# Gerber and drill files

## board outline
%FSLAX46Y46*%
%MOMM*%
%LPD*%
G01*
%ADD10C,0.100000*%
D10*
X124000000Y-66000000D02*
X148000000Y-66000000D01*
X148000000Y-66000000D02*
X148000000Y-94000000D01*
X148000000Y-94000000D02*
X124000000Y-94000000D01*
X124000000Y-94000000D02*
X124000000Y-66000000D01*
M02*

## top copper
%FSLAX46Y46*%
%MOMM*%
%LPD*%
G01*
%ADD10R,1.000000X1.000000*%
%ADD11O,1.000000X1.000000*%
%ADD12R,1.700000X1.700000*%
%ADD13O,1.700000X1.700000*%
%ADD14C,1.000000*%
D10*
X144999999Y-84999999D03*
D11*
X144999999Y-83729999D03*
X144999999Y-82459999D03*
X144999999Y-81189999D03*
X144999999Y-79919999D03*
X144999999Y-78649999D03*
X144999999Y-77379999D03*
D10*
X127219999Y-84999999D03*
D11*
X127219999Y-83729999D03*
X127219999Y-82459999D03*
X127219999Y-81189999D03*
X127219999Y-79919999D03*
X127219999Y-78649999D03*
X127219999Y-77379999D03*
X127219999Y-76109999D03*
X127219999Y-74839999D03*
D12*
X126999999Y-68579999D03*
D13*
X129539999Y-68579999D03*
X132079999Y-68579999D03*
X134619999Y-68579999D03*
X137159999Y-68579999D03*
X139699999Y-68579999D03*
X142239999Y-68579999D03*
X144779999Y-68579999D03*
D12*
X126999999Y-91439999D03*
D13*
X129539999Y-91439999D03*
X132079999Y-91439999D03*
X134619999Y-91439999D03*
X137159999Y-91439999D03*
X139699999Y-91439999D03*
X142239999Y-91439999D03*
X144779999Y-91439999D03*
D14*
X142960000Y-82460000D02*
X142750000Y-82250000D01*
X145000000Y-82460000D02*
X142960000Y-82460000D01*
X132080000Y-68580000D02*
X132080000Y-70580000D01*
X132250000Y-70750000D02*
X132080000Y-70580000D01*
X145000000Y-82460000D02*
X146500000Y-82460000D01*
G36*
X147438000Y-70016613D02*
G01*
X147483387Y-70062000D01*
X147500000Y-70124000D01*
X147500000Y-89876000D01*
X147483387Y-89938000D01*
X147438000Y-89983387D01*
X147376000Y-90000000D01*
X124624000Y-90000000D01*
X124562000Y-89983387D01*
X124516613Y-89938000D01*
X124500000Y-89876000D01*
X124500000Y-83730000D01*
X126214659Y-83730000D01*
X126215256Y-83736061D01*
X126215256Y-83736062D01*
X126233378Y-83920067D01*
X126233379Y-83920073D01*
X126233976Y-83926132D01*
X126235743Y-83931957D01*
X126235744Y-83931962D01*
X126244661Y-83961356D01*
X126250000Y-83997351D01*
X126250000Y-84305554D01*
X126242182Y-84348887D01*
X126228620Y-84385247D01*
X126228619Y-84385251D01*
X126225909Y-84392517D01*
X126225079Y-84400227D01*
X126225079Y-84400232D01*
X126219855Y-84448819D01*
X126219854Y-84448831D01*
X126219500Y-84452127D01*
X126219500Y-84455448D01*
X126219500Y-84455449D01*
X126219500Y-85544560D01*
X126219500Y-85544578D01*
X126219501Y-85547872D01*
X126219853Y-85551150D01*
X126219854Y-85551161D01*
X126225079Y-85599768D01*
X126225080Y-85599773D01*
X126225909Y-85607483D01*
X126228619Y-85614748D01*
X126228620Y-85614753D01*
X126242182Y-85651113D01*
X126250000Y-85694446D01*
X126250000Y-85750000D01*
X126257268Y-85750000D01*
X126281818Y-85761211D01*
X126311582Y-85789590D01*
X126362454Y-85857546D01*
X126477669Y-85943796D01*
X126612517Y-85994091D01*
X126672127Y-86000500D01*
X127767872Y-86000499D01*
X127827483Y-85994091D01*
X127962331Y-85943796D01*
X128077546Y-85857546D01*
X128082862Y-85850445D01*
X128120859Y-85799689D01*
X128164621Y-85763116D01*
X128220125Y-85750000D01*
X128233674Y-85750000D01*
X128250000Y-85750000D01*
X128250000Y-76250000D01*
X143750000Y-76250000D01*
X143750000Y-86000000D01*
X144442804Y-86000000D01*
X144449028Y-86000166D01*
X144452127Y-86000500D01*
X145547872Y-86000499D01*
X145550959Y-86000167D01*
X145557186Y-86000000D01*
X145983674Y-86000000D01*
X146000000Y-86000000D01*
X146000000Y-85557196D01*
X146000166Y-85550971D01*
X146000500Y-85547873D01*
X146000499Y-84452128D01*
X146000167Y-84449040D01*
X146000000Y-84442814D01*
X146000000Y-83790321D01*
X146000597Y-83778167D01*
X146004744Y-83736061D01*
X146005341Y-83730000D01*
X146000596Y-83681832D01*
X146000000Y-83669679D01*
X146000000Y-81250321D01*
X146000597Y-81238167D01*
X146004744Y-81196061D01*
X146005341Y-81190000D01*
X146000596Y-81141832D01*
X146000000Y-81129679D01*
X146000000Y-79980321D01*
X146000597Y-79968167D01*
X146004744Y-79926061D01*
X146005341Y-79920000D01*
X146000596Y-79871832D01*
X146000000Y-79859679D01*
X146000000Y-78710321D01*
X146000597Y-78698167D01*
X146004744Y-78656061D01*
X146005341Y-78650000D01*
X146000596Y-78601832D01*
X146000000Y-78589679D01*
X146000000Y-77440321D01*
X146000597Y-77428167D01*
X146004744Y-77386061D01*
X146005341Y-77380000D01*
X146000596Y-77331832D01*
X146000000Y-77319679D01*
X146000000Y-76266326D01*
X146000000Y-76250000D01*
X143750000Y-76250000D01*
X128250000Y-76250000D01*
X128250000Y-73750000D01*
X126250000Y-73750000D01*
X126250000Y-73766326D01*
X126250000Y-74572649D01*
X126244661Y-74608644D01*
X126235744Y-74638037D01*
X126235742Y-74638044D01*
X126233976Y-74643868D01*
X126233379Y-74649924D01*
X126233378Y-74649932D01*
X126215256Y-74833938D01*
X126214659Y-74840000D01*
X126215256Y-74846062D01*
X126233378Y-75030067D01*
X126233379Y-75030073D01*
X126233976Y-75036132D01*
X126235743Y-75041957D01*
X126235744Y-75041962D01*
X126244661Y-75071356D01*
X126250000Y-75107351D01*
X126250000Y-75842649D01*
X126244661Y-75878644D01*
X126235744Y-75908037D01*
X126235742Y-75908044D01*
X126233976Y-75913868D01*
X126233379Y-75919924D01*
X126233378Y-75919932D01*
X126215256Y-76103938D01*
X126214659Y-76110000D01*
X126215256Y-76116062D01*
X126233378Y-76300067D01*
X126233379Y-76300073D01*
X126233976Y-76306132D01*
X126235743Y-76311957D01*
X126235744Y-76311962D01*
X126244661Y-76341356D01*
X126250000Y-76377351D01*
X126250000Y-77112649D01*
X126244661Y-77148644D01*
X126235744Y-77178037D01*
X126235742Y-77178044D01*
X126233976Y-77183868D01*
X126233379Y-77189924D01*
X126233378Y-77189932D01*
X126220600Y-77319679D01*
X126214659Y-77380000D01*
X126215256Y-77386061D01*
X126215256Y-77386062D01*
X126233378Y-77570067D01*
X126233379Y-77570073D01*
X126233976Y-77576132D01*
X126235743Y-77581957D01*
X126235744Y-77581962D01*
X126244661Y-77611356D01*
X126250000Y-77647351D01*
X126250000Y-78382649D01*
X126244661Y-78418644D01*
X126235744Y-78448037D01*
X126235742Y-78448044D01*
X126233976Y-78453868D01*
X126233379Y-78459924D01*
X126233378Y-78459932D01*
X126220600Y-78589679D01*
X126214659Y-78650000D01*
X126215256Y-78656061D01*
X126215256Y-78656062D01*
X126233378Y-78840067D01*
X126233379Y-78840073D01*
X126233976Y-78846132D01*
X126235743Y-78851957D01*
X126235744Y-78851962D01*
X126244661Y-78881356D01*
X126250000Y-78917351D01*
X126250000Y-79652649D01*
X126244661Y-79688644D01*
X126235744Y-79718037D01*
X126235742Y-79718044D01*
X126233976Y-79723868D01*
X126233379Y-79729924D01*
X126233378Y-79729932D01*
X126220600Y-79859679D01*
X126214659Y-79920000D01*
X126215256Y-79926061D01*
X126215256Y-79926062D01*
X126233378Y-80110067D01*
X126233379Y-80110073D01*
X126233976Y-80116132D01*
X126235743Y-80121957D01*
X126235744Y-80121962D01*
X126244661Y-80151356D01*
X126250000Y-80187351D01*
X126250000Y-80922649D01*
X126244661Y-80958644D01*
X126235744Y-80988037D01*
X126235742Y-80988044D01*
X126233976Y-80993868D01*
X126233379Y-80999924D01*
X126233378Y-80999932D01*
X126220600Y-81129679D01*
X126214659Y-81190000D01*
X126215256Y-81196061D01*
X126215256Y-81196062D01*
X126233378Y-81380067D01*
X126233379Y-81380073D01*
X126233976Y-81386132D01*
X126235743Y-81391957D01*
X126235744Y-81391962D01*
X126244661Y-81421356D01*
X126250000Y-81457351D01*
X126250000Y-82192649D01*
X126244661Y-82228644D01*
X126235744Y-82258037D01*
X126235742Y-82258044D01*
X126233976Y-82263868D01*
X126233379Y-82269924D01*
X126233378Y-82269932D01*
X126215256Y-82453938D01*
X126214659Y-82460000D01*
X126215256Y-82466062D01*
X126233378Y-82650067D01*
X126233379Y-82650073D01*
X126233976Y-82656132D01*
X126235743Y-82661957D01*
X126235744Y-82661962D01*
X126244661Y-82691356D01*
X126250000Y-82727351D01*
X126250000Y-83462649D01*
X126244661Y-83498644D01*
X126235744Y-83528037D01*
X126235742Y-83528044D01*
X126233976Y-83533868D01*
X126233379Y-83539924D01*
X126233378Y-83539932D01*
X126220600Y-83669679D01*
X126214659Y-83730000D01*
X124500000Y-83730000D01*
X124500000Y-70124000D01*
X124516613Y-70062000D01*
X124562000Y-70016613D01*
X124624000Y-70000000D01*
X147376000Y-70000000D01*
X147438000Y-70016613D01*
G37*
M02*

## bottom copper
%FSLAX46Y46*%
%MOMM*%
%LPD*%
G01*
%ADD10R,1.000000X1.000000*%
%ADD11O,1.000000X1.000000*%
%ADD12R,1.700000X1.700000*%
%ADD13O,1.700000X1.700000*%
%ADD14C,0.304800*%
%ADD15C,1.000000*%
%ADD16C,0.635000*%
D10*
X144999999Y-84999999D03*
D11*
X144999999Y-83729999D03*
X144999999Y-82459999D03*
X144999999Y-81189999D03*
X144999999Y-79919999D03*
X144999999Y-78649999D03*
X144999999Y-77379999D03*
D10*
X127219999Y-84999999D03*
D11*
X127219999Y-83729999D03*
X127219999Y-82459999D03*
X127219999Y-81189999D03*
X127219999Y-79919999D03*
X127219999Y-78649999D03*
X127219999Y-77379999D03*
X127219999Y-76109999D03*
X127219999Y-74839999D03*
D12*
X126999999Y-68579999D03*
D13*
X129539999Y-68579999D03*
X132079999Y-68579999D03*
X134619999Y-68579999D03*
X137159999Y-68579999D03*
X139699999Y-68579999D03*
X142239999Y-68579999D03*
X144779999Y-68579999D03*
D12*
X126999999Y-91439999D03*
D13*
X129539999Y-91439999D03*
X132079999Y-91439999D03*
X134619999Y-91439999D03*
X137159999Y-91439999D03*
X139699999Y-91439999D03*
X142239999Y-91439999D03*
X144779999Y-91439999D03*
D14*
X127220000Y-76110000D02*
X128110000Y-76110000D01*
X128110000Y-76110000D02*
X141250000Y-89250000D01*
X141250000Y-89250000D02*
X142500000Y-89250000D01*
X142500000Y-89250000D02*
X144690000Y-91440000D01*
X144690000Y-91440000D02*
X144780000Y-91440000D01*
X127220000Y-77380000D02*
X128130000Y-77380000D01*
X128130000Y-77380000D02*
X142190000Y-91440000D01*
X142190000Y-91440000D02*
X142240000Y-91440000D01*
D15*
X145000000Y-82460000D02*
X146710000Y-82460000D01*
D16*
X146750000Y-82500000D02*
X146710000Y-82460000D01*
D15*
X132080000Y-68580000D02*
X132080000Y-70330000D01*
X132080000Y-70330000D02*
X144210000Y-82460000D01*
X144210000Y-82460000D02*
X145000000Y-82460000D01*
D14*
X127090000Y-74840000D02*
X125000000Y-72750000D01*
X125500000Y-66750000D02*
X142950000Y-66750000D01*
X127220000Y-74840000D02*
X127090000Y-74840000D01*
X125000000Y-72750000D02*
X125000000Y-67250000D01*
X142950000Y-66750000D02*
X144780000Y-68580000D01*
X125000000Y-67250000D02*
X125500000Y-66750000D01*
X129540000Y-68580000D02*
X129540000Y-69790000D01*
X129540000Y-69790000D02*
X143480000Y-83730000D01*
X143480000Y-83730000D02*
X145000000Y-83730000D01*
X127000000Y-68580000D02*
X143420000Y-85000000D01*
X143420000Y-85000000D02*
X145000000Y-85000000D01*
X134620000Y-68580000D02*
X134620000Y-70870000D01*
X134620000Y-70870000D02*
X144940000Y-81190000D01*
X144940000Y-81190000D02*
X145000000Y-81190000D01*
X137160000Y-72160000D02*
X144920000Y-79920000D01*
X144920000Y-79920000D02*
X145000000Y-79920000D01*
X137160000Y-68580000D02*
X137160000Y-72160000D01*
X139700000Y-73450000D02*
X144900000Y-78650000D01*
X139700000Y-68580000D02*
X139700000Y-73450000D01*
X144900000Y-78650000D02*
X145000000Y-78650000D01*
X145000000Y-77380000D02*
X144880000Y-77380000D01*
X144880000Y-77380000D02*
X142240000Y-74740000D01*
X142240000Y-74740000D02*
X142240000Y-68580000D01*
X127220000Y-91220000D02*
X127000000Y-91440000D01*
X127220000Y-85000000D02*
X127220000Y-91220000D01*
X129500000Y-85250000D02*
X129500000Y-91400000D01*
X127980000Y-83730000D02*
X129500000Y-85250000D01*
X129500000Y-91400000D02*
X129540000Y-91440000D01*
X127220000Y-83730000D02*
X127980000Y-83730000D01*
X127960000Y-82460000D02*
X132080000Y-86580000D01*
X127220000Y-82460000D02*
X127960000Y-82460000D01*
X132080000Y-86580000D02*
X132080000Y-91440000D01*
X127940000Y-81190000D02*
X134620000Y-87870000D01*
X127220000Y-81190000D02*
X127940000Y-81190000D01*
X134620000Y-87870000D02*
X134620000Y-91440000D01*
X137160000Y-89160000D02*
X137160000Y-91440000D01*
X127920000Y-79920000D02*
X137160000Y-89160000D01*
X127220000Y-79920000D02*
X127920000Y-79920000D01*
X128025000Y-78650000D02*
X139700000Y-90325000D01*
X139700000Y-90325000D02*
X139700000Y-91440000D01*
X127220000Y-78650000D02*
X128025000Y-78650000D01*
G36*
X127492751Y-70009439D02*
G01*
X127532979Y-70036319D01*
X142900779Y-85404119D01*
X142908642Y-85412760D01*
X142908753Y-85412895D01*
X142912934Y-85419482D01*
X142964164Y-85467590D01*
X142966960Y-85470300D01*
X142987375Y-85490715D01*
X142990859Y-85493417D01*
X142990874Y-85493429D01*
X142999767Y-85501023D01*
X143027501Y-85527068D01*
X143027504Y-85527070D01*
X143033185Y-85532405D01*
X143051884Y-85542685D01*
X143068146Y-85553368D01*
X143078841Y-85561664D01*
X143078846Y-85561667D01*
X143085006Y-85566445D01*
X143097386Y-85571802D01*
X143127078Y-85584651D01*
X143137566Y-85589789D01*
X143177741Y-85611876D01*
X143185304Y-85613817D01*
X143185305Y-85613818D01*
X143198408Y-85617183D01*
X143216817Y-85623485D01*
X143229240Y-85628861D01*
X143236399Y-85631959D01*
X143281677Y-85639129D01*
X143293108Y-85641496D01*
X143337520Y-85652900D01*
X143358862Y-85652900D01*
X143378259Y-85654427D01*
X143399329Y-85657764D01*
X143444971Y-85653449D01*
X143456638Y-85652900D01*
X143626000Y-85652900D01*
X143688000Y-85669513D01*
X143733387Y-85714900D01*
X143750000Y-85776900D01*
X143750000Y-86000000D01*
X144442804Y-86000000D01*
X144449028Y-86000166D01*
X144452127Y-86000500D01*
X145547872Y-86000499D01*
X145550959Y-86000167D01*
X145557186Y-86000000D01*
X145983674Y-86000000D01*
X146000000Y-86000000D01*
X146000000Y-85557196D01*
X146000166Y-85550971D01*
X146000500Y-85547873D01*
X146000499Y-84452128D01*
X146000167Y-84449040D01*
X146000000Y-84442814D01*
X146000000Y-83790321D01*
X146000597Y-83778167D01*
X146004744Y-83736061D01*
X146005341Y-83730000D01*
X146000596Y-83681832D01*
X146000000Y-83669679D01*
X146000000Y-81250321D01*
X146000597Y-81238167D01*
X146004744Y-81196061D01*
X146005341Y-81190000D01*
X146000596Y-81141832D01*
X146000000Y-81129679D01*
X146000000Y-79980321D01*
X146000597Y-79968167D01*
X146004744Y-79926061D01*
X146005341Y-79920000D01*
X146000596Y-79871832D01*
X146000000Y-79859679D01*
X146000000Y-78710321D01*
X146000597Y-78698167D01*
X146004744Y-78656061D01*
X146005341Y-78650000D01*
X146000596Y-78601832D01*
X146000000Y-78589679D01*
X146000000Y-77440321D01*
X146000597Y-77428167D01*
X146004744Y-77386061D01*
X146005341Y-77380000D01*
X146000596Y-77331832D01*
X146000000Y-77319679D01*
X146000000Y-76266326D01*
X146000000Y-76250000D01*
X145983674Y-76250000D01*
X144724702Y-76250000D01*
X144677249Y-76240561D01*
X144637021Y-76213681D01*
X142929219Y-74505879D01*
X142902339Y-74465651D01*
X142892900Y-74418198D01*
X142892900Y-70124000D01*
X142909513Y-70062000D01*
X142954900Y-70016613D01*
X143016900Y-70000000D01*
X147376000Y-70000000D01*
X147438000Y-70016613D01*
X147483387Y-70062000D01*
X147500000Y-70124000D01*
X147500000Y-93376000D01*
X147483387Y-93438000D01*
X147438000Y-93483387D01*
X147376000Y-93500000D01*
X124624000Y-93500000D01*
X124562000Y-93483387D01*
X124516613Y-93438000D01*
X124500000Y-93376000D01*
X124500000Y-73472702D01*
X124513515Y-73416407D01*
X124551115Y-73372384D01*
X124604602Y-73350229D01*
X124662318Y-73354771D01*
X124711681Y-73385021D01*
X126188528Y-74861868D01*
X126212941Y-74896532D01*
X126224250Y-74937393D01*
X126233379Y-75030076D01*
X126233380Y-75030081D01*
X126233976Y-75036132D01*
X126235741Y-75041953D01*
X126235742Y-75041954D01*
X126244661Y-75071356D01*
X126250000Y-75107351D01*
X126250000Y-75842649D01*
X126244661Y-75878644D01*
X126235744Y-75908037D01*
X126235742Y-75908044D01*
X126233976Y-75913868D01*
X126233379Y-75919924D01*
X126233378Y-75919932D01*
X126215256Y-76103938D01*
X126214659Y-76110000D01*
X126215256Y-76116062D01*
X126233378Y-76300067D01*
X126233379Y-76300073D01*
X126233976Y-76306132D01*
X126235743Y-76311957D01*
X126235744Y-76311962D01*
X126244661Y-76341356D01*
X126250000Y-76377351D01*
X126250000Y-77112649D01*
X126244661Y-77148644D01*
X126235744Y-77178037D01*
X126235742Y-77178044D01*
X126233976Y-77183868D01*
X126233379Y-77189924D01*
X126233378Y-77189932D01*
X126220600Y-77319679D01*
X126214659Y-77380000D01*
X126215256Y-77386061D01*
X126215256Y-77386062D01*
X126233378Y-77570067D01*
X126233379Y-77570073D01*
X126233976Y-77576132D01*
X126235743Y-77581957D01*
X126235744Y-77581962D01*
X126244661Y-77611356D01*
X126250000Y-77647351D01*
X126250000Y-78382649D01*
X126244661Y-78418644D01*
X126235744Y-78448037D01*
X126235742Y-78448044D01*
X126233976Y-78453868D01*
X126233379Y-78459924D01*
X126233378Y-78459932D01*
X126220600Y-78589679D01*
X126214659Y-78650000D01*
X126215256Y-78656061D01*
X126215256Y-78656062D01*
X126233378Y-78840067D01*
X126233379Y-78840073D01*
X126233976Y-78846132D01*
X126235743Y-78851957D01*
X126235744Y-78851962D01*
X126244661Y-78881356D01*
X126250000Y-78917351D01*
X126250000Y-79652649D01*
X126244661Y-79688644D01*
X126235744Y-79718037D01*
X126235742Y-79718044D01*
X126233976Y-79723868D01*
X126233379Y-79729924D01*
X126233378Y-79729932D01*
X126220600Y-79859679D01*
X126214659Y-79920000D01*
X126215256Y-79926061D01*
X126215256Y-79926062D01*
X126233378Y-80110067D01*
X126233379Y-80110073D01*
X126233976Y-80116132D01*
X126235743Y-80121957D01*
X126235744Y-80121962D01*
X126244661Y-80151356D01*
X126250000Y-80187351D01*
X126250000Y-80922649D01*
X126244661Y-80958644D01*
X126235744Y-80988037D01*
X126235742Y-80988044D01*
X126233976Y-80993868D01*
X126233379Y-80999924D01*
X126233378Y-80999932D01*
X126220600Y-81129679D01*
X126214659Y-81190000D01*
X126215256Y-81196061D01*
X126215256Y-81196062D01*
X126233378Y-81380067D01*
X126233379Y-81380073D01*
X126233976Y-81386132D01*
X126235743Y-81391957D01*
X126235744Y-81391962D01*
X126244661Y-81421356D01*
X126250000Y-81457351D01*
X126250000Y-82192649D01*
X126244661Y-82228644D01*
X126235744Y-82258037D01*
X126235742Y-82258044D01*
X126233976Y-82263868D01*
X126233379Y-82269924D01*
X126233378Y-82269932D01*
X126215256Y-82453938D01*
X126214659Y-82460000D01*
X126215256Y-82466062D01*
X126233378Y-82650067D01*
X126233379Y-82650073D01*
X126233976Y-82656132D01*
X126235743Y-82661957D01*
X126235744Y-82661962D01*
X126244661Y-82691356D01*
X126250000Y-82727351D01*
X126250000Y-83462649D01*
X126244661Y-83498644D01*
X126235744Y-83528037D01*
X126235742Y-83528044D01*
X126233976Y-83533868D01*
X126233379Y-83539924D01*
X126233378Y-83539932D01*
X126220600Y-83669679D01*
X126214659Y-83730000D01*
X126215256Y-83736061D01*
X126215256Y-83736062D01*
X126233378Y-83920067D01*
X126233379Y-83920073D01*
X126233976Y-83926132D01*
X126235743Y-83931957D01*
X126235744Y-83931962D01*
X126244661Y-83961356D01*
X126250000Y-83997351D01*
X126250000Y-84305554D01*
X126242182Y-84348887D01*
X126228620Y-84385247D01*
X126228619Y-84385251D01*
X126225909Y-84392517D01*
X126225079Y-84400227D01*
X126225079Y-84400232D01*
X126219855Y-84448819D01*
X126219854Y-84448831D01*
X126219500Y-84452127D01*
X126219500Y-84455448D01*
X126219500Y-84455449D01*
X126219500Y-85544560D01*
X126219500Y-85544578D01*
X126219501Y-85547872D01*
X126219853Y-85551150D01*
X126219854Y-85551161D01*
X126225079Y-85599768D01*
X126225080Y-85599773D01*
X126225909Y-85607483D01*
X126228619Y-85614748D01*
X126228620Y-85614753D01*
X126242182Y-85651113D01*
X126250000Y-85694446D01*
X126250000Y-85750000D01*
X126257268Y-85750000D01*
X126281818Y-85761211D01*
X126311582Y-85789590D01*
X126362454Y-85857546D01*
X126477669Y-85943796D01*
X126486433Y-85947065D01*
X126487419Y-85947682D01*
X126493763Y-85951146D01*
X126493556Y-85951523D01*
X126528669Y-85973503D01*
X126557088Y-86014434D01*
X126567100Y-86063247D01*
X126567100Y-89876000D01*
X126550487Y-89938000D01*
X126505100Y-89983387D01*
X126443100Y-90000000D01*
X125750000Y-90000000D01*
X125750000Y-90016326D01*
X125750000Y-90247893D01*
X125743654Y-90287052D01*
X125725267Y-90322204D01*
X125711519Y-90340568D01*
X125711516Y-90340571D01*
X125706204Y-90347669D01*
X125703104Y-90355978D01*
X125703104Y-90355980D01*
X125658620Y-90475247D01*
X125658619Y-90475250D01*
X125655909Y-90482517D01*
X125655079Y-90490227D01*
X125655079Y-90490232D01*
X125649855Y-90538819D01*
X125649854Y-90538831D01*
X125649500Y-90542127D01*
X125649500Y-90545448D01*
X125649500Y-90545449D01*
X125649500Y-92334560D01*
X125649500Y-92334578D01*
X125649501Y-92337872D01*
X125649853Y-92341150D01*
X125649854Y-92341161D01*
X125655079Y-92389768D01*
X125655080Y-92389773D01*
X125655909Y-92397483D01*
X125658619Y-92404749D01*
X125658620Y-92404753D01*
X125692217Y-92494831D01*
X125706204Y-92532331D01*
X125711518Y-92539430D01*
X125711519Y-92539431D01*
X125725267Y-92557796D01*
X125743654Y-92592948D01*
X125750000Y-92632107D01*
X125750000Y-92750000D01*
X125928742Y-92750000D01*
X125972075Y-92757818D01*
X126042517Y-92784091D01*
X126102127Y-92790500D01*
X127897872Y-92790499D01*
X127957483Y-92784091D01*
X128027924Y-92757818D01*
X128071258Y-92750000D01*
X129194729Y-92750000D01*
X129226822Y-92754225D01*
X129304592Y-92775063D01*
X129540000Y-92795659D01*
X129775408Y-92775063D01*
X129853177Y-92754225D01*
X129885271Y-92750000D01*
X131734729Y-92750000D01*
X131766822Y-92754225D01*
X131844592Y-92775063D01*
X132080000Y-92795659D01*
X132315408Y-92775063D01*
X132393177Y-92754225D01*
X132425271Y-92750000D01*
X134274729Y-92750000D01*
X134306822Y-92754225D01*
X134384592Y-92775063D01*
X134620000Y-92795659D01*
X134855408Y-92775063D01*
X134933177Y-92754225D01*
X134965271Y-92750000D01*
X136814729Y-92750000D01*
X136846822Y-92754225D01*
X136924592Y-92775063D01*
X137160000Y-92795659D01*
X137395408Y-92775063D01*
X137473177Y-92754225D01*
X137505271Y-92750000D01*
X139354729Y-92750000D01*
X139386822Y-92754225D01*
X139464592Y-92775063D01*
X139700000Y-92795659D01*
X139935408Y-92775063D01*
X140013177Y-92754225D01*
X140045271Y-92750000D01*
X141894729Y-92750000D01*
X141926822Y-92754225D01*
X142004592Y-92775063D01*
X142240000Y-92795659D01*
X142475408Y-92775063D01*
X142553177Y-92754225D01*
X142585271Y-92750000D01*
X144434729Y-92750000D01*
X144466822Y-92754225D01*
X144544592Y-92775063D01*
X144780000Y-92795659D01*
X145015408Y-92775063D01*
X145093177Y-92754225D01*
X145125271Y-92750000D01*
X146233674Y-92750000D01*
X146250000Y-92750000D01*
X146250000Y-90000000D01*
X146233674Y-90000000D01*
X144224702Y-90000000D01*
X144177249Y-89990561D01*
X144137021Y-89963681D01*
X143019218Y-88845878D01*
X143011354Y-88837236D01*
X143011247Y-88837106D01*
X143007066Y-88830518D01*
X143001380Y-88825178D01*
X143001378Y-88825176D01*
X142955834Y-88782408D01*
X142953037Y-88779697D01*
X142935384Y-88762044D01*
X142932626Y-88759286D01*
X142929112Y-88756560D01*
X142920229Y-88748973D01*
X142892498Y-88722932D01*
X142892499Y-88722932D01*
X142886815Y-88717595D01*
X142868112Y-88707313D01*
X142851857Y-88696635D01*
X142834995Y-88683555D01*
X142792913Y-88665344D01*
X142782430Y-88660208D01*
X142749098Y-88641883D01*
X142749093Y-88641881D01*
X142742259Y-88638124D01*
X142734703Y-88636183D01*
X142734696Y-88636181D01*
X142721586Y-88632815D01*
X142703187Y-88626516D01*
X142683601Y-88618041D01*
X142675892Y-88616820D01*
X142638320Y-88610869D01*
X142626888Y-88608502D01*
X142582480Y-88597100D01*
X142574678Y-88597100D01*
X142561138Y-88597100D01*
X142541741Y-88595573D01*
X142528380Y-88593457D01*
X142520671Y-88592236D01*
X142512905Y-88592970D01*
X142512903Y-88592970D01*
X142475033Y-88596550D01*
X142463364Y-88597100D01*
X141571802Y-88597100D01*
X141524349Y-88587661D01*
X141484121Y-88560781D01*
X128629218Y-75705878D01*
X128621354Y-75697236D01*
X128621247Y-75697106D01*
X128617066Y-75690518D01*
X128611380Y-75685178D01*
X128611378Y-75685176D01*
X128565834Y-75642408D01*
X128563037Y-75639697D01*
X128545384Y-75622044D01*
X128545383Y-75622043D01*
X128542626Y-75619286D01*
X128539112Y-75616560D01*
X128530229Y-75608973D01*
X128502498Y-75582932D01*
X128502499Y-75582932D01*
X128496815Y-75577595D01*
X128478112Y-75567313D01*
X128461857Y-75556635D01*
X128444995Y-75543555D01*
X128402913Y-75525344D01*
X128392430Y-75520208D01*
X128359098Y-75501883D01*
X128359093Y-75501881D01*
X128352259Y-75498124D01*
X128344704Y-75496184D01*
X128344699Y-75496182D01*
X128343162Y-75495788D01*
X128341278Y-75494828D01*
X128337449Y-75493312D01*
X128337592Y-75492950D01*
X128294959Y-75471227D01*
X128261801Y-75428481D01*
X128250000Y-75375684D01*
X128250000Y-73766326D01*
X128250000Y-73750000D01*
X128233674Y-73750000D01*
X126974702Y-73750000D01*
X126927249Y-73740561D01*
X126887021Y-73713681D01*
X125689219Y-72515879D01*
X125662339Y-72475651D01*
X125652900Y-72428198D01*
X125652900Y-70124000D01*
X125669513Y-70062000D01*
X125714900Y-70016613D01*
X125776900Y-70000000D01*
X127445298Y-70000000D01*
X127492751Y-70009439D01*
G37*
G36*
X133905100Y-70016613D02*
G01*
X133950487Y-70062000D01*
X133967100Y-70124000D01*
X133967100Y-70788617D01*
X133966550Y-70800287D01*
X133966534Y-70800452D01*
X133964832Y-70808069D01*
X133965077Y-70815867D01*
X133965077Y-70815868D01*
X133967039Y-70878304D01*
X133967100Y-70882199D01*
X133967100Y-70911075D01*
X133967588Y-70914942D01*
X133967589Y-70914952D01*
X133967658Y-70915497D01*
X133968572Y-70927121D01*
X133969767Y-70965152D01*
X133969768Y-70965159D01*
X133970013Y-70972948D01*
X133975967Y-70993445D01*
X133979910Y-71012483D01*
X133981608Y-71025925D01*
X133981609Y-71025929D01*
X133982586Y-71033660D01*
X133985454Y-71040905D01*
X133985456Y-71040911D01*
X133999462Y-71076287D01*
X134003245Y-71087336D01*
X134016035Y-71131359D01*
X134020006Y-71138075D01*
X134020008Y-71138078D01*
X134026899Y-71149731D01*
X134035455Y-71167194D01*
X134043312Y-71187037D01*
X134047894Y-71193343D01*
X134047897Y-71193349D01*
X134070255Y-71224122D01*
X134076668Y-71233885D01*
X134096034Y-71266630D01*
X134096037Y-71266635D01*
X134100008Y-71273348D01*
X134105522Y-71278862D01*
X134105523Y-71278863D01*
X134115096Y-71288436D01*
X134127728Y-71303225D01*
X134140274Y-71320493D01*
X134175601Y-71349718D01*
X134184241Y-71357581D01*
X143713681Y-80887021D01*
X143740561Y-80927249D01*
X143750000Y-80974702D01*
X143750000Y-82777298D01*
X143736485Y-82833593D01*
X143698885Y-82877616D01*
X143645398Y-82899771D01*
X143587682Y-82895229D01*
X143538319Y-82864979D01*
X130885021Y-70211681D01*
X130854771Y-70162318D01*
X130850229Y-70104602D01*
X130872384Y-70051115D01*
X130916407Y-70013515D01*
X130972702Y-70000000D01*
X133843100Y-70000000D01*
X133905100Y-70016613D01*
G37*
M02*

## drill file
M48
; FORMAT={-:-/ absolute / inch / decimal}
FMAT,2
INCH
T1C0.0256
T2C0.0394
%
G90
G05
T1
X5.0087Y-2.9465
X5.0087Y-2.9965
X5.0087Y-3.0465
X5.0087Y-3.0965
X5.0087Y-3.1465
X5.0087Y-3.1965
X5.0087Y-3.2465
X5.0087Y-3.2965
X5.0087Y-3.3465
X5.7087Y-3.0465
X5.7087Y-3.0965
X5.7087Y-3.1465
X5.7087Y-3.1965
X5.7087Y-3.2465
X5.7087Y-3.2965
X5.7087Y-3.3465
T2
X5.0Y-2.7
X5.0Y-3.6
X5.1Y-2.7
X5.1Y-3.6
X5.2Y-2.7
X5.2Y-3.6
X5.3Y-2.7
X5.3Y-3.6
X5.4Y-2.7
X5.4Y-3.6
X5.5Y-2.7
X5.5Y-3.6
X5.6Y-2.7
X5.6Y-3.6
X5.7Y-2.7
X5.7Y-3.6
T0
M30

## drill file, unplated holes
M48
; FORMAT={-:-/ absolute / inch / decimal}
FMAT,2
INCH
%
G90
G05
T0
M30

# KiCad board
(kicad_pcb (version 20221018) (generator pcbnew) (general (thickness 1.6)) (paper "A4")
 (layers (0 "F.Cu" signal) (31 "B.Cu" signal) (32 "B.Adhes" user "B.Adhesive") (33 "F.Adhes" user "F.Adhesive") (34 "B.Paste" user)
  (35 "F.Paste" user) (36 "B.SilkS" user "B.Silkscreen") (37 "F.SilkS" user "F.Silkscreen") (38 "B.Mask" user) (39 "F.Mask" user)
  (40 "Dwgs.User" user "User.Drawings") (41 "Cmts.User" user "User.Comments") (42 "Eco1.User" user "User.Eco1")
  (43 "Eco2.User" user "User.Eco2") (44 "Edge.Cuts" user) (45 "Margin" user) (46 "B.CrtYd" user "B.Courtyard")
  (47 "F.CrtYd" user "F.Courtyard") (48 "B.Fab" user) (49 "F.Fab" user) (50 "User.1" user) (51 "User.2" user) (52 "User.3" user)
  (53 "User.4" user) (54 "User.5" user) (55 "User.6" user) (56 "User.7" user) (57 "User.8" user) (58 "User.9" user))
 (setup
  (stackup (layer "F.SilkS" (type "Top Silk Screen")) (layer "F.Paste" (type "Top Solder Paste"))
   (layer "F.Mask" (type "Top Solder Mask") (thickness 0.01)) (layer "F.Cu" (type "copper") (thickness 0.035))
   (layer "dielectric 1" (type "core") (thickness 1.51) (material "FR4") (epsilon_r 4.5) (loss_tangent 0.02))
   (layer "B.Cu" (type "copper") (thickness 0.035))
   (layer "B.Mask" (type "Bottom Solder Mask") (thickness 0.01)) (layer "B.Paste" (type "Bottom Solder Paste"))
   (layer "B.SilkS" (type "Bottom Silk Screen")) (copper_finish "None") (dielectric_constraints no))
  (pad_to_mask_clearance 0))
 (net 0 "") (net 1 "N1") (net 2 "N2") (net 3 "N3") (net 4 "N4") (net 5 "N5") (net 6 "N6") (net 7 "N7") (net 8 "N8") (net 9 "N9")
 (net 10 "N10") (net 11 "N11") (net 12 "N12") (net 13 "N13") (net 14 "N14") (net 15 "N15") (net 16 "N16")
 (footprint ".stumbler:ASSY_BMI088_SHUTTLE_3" (layer "F.Cu") (at 136.11 79.92)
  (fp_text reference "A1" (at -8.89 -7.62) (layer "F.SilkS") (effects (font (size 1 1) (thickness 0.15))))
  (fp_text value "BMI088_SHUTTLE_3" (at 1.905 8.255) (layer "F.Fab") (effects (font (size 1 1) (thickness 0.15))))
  (pad "11" thru_hole rect (at 8.89 5.08 180) (size 1 1) (drill 0.65) (layers "*.Cu" "*.Mask") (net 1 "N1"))
  (pad "12" thru_hole oval (at 8.89 3.81 180) (size 1 1) (drill 0.65) (layers "*.Cu" "*.Mask") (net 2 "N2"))
  (pad "13" thru_hole oval (at 8.89 2.54 180) (size 1 1) (drill 0.65) (layers "*.Cu" "*.Mask") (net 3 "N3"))
  (pad "14" thru_hole oval (at 8.89 1.27 180) (size 1 1) (drill 0.65) (layers "*.Cu" "*.Mask") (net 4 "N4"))
  (pad "15" thru_hole oval (at 8.89 0 180) (size 1 1) (drill 0.65) (layers "*.Cu" "*.Mask") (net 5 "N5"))
  (pad "16" thru_hole oval (at 8.89 -1.27 180) (size 1 1) (drill 0.65) (layers "*.Cu" "*.Mask") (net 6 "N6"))
  (pad "17" thru_hole oval (at 8.89 -2.54 180) (size 1 1) (drill 0.65) (layers "*.Cu" "*.Mask") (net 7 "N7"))
  (pad "21" thru_hole rect (at -8.89 5.08 180) (size 1 1) (drill 0.65) (layers "*.Cu" "*.Mask") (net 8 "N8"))
  (pad "22" thru_hole oval (at -8.89 3.81 180) (size 1 1) (drill 0.65) (layers "*.Cu" "*.Mask") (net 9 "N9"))
  (pad "23" thru_hole oval (at -8.89 2.54 180) (size 1 1) (drill 0.65) (layers "*.Cu" "*.Mask") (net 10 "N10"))
  (pad "24" thru_hole oval (at -8.89 1.27 180) (size 1 1) (drill 0.65) (layers "*.Cu" "*.Mask") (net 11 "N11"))
  (pad "25" thru_hole oval (at -8.89 0 180) (size 1 1) (drill 0.65) (layers "*.Cu" "*.Mask") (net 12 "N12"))
  (pad "26" thru_hole oval (at -8.89 -1.27 180) (size 1 1) (drill 0.65) (layers "*.Cu" "*.Mask") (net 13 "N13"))
  (pad "27" thru_hole oval (at -8.89 -2.54 180) (size 1 1) (drill 0.65) (layers "*.Cu" "*.Mask") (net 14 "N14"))
  (pad "28" thru_hole oval (at -8.89 -3.81 180) (size 1 1) (drill 0.65) (layers "*.Cu" "*.Mask") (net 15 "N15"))
  (pad "29" thru_hole oval (at -8.89 -5.08 180) (size 1 1) (drill 0.65) (layers "*.Cu" "*.Mask") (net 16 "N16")))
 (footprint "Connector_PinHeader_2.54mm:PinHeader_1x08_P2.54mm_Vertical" (layer "B.Cu") (at 127 68.58 -90)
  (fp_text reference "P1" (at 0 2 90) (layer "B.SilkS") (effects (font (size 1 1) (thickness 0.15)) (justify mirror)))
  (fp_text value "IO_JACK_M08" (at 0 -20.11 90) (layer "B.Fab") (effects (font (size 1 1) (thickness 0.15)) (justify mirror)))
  (pad "1" thru_hole rect (at 0 0 270) (size 1.7 1.7) (drill 1) (layers "*.Cu" "*.Mask") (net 1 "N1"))
  (pad "2" thru_hole oval (at 0 -2.54 270) (size 1.7 1.7) (drill 1) (layers "*.Cu" "*.Mask") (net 2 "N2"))
  (pad "3" thru_hole oval (at 0 -5.08 270) (size 1.7 1.7) (drill 1) (layers "*.Cu" "*.Mask") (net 3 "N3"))
  (pad "4" thru_hole oval (at 0 -7.62 270) (size 1.7 1.7) (drill 1) (layers "*.Cu" "*.Mask") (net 4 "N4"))
  (pad "5" thru_hole oval (at 0 -10.16 270) (size 1.7 1.7) (drill 1) (layers "*.Cu" "*.Mask") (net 5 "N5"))
  (pad "6" thru_hole oval (at 0 -12.7 270) (size 1.7 1.7) (drill 1) (layers "*.Cu" "*.Mask") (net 6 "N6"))
  (pad "7" thru_hole oval (at 0 -15.24 270) (size 1.7 1.7) (drill 1) (layers "*.Cu" "*.Mask") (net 7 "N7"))
  (pad "8" thru_hole oval (at 0 -17.78 270) (size 1.7 1.7) (drill 1) (layers "*.Cu" "*.Mask") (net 16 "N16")))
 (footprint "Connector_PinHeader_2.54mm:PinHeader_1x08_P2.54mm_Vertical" (layer "B.Cu") (at 127 91.44 -90)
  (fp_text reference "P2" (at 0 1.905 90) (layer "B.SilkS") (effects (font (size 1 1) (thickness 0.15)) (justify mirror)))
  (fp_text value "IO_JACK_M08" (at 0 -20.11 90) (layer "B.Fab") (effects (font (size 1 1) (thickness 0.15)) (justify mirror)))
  (pad "1" thru_hole rect (at 0 0 270) (size 1.7 1.7) (drill 1) (layers "*.Cu" "*.Mask") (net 8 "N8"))
  (pad "2" thru_hole oval (at 0 -2.54 270) (size 1.7 1.7) (drill 1) (layers "*.Cu" "*.Mask") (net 9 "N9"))
  (pad "3" thru_hole oval (at 0 -5.08 270) (size 1.7 1.7) (drill 1) (layers "*.Cu" "*.Mask") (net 10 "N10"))
  (pad "4" thru_hole oval (at 0 -7.62 270) (size 1.7 1.7) (drill 1) (layers "*.Cu" "*.Mask") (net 11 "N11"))
  (pad "5" thru_hole oval (at 0 -10.16 270) (size 1.7 1.7) (drill 1) (layers "*.Cu" "*.Mask") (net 12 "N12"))
  (pad "6" thru_hole oval (at 0 -12.7 270) (size 1.7 1.7) (drill 1) (layers "*.Cu" "*.Mask") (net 13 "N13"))
  (pad "7" thru_hole oval (at 0 -15.24 270) (size 1.7 1.7) (drill 1) (layers "*.Cu" "*.Mask") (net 14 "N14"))
  (pad "8" thru_hole oval (at 0 -17.78 270) (size 1.7 1.7) (drill 1) (layers "*.Cu" "*.Mask") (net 15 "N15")))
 (gr_rect (start 124 66) (end 148 94) (stroke (width 0.1) (type default)) (fill none) (layer "Edge.Cuts"))
 (segment (start 143.42 85) (end 145 85) (width 0.3048) (layer "B.Cu") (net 1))
 (segment (start 127 68.58) (end 143.42 85) (width 0.3048) (layer "B.Cu") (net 1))
 (segment (start 129.54 69.79) (end 143.48 83.73) (width 0.3048) (layer "B.Cu") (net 2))
 (segment (start 143.48 83.73) (end 145 83.73) (width 0.3048) (layer "B.Cu") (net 2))
 (segment (start 129.54 68.58) (end 129.54 69.79) (width 0.3048) (layer "B.Cu") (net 2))
 (segment (start 142.96 82.46) (end 142.75 82.25) (width 1) (layer "F.Cu") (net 3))
 (segment (start 132.25 70.75) (end 132.08 70.58) (width 1) (layer "F.Cu") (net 3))
 (segment (start 132.08 68.58) (end 132.08 70.58) (width 1) (layer "F.Cu") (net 3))
 (segment (start 145 82.46) (end 142.96 82.46) (width 1) (layer "F.Cu") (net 3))
 (segment (start 145 82.46) (end 146.5 82.46) (width 1) (layer "F.Cu") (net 3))
 (segment (start 132.08 68.58) (end 132.08 70.33) (width 1) (layer "B.Cu") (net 3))
 (segment (start 144.21 82.46) (end 145 82.46) (width 1) (layer "B.Cu") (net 3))
 (segment (start 146.75 82.5) (end 146.71 82.46) (width 0.635) (layer "B.Cu") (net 3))
 (segment (start 132.08 70.33) (end 144.21 82.46) (width 1) (layer "B.Cu") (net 3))
 (segment (start 145 82.46) (end 146.71 82.46) (width 1) (layer "B.Cu") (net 3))
 (segment (start 134.62 68.58) (end 134.62 70.87) (width 0.3048) (layer "B.Cu") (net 4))
 (segment (start 134.62 70.87) (end 144.94 81.19) (width 0.3048) (layer "B.Cu") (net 4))
 (segment (start 144.94 81.19) (end 145 81.19) (width 0.3048) (layer "B.Cu") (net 4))
 (segment (start 137.16 72.16) (end 144.92 79.92) (width 0.3048) (layer "B.Cu") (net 5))
 (segment (start 144.92 79.92) (end 145 79.92) (width 0.3048) (layer "B.Cu") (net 5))
 (segment (start 137.16 68.58) (end 137.16 72.16) (width 0.3048) (layer "B.Cu") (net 5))
 (segment (start 139.7 73.45) (end 144.9 78.65) (width 0.3048) (layer "B.Cu") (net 6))
 (segment (start 139.7 68.58) (end 139.7 73.45) (width 0.3048) (layer "B.Cu") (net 6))
 (segment (start 144.9 78.65) (end 145 78.65) (width 0.3048) (layer "B.Cu") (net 6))
 (segment (start 145 77.38) (end 144.88 77.38) (width 0.3048) (layer "B.Cu") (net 7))
 (segment (start 144.88 77.38) (end 142.24 74.74) (width 0.3048) (layer "B.Cu") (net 7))
 (segment (start 142.24 74.74) (end 142.24 68.58) (width 0.3048) (layer "B.Cu") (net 7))
 (segment (start 127.22 91.22) (end 127 91.44) (width 0.3048) (layer "B.Cu") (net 8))
 (segment (start 127.22 85) (end 127.22 91.22) (width 0.3048) (layer "B.Cu") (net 8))
 (segment (start 129.5 85.25) (end 129.5 91.4) (width 0.3048) (layer "B.Cu") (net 9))
 (segment (start 127.98 83.73) (end 129.5 85.25) (width 0.3048) (layer "B.Cu") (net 9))
 (segment (start 129.5 91.4) (end 129.54 91.44) (width 0.3048) (layer "B.Cu") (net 9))
 (segment (start 127.22 83.73) (end 127.98 83.73) (width 0.3048) (layer "B.Cu") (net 9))
 (segment (start 127.96 82.46) (end 132.08 86.58) (width 0.3048) (layer "B.Cu") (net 10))
 (segment (start 127.22 82.46) (end 127.96 82.46) (width 0.3048) (layer "B.Cu") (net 10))
 (segment (start 132.08 86.58) (end 132.08 91.44) (width 0.3048) (layer "B.Cu") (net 10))
 (segment (start 127.94 81.19) (end 134.62 87.87) (width 0.3048) (layer "B.Cu") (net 11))
 (segment (start 127.22 81.19) (end 127.94 81.19) (width 0.3048) (layer "B.Cu") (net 11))
 (segment (start 134.62 87.87) (end 134.62 91.44) (width 0.3048) (layer "B.Cu") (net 11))
 (segment (start 137.16 89.16) (end 137.16 91.44) (width 0.3048) (layer "B.Cu") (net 12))
 (segment (start 127.92 79.92) (end 137.16 89.16) (width 0.3048) (layer "B.Cu") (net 12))
 (segment (start 127.22 79.92) (end 127.92 79.92) (width 0.3048) (layer "B.Cu") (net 12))
 (segment (start 128.025 78.65) (end 139.7 90.325) (width 0.3048) (layer "B.Cu") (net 13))
 (segment (start 139.7 90.325) (end 139.7 91.44) (width 0.3048) (layer "B.Cu") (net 13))
 (segment (start 127.22 78.65) (end 128.025 78.65) (width 0.3048) (layer "B.Cu") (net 13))
 (segment (start 127.22 77.38) (end 128.13 77.38) (width 0.3048) (layer "B.Cu") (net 14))
 (segment (start 142.19 91.44) (end 142.24 91.44) (width 0.3048) (layer "B.Cu") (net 14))
 (segment (start 128.13 77.38) (end 142.19 91.44) (width 0.3048) (layer "B.Cu") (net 14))
 (segment (start 128.11 76.11) (end 141.25 89.25) (width 0.3048) (layer "B.Cu") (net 15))
 (segment (start 144.69 91.44) (end 144.78 91.44) (width 0.3048) (layer "B.Cu") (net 15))
 (segment (start 127.22 76.11) (end 128.11 76.11) (width 0.3048) (layer "B.Cu") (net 15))
 (segment (start 142.5 89.25) (end 144.69 91.44) (width 0.3048) (layer "B.Cu") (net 15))
 (segment (start 141.25 89.25) (end 142.5 89.25) (width 0.3048) (layer "B.Cu") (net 15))
 (segment (start 142.95 66.75) (end 144.78 68.58) (width 0.3048) (layer "B.Cu") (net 16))
 (segment (start 125.5 66.75) (end 142.95 66.75) (width 0.3048) (layer "B.Cu") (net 16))
 (segment (start 127.22 74.84) (end 127.09 74.84) (width 0.3048) (layer "B.Cu") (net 16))
 (segment (start 125 72.75) (end 125 67.25) (width 0.3048) (layer "B.Cu") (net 16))
 (segment (start 127.09 74.84) (end 125 72.75) (width 0.3048) (layer "B.Cu") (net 16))
 (segment (start 125 67.25) (end 125.5 66.75) (width 0.3048) (layer "B.Cu") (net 16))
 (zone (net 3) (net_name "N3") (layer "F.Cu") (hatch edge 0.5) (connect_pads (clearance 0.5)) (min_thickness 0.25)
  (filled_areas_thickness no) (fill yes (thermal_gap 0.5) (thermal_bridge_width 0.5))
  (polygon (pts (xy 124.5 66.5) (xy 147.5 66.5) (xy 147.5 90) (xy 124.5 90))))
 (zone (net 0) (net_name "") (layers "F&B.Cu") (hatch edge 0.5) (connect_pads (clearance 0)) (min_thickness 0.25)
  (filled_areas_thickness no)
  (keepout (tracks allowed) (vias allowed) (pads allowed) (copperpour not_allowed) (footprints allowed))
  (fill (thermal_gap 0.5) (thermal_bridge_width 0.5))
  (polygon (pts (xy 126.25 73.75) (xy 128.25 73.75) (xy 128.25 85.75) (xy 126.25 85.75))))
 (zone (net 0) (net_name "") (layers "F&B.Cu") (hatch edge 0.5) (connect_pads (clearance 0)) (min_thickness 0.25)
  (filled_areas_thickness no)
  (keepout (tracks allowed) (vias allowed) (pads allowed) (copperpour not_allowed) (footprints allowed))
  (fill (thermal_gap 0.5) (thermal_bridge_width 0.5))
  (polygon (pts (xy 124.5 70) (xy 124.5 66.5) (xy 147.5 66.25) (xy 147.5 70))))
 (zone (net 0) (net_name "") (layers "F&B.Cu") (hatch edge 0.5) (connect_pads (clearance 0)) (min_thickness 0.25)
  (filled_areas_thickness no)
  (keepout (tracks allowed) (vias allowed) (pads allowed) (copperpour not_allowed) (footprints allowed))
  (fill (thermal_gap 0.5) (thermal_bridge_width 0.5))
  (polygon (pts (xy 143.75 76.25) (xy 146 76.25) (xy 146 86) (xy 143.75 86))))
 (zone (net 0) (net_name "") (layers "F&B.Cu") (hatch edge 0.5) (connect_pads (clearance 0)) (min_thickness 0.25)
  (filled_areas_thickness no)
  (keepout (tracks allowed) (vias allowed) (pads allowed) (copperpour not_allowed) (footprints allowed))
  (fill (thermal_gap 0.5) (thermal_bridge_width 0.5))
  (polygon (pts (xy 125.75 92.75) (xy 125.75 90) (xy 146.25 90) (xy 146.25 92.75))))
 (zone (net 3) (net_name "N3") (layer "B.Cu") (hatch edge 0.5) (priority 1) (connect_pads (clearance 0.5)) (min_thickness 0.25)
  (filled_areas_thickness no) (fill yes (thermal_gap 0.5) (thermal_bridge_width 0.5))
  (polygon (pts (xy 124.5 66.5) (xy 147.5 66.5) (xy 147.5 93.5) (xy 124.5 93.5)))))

